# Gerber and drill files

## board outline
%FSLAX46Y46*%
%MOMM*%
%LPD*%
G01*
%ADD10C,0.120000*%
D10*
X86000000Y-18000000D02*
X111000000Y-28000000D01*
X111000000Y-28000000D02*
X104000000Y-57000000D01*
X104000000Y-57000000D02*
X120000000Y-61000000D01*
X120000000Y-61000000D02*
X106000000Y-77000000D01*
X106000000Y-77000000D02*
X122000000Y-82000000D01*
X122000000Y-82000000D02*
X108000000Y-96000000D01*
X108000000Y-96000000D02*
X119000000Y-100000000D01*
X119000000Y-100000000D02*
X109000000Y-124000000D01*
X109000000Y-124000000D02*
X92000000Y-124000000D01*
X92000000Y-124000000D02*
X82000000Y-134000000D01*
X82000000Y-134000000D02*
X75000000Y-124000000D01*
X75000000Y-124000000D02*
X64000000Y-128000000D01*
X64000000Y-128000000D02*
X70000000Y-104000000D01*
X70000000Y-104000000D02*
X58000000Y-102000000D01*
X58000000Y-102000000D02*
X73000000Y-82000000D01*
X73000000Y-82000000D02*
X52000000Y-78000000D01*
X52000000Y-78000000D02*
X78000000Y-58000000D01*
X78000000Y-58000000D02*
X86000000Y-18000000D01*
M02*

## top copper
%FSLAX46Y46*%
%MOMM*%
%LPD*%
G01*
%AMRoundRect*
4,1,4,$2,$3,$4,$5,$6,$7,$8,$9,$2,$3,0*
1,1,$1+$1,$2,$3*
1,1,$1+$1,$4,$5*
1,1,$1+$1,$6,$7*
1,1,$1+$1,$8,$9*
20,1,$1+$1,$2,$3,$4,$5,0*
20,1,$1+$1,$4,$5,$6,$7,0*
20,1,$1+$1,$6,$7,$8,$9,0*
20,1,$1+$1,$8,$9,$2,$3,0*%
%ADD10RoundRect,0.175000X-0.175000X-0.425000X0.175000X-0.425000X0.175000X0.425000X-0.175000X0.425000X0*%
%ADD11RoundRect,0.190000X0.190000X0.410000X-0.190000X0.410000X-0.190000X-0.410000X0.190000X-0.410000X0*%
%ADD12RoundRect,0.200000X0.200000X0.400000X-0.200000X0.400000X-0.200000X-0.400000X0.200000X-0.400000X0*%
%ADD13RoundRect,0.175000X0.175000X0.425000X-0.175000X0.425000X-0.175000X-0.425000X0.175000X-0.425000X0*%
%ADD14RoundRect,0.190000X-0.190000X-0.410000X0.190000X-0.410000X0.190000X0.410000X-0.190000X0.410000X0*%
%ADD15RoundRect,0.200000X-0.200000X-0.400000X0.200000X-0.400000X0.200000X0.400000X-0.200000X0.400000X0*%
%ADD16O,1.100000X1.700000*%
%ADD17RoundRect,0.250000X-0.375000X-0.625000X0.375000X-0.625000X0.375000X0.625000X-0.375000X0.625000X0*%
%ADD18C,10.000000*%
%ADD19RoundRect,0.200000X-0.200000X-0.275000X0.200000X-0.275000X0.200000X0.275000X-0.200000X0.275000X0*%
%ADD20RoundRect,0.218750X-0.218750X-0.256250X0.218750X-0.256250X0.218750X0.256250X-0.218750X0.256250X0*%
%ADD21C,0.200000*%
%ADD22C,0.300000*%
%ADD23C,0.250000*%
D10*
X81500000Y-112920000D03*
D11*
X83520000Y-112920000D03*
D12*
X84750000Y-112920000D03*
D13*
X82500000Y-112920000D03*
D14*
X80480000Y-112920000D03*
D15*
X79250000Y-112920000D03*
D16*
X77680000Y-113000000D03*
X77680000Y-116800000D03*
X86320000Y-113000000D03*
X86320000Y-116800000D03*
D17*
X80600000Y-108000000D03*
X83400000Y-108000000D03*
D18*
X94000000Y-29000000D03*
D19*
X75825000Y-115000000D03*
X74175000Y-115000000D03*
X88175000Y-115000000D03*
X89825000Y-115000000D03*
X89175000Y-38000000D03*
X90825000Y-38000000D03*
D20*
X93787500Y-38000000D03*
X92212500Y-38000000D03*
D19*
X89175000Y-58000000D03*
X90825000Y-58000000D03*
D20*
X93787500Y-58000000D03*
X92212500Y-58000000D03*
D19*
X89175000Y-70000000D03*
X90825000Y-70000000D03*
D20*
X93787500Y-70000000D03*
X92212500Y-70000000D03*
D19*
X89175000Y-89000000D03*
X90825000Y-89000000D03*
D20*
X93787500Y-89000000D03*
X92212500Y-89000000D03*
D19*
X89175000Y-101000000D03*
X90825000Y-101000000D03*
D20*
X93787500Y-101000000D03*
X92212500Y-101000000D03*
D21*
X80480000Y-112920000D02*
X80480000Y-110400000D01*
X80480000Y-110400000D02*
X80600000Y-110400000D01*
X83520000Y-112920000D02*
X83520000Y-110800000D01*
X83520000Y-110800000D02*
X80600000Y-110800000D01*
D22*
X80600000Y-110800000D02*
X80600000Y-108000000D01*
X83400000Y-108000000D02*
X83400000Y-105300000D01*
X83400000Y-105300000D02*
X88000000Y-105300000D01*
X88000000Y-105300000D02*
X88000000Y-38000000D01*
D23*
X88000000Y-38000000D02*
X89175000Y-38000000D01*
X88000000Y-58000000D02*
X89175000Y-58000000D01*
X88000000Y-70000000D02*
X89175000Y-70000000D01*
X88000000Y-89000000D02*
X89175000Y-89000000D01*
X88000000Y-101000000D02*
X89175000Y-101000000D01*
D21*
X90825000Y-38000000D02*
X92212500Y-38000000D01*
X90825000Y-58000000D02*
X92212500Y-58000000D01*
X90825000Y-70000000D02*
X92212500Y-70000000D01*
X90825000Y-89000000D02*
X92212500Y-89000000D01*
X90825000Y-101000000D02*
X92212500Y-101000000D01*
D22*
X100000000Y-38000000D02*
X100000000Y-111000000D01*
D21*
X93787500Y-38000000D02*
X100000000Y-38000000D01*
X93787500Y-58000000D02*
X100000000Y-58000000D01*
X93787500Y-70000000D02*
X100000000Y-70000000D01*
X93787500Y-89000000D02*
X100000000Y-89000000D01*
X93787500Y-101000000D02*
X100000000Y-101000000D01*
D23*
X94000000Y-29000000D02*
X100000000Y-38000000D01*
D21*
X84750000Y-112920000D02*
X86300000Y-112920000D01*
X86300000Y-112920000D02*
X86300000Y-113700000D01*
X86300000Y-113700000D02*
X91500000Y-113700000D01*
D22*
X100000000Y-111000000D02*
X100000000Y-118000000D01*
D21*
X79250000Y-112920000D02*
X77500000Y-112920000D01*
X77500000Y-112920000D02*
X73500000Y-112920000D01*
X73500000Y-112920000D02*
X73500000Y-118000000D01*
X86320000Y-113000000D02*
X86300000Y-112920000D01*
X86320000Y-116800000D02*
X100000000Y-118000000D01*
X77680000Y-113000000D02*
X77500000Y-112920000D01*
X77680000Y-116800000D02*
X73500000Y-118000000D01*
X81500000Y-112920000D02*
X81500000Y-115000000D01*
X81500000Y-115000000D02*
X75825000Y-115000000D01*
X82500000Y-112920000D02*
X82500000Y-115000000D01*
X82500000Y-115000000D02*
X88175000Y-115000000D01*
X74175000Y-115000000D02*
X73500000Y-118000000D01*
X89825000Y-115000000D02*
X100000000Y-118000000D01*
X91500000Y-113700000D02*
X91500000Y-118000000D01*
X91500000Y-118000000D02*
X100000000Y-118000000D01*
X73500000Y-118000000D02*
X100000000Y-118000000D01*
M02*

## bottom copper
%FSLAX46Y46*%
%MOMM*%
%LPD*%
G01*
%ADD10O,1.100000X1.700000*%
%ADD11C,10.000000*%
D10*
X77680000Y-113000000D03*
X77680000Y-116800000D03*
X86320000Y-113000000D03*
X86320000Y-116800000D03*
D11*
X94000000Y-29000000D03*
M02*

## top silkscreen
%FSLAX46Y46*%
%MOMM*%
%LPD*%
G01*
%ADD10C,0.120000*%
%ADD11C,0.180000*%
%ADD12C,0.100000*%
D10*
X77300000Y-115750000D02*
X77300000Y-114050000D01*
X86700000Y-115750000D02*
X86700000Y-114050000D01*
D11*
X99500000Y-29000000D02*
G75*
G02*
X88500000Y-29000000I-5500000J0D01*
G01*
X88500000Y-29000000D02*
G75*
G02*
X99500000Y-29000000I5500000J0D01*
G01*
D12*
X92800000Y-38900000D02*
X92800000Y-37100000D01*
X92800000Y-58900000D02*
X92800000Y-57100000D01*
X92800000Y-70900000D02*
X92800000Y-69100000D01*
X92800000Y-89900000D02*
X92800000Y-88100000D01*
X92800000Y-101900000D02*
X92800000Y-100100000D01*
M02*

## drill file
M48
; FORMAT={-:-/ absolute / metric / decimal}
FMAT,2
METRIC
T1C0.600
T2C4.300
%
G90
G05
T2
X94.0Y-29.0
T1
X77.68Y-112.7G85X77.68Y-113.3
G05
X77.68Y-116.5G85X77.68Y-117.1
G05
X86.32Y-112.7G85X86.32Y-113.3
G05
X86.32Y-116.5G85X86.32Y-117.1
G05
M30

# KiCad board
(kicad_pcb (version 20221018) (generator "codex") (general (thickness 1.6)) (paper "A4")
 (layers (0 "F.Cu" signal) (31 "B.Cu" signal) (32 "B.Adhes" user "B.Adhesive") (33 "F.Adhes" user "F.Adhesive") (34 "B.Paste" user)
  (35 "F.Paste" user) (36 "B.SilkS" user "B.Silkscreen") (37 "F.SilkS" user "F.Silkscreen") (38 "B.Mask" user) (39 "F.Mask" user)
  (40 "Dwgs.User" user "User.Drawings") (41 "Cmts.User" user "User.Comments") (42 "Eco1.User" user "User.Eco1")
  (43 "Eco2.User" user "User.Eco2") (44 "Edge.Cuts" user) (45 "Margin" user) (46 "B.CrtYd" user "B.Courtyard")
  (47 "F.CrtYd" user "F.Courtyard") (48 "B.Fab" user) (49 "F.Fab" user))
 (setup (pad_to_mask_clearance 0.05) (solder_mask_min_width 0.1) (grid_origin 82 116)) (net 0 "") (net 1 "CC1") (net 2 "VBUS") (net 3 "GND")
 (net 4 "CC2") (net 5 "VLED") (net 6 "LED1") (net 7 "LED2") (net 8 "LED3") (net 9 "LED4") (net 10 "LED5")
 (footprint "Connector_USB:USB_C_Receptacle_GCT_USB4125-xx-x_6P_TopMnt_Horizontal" (layer "F.Cu") (at 82 116)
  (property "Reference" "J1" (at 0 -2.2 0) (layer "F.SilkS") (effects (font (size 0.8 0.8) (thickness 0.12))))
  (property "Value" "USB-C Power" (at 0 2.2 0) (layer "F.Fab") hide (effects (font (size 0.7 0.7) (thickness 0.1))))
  (fp_line (start -4.7 -0.25) (end -4.7 -1.95) (stroke (width 0.12) (type solid)) (layer "F.SilkS"))
  (fp_line (start 4.7 -0.25) (end 4.7 -1.95) (stroke (width 0.12) (type solid)) (layer "F.SilkS"))
  (pad "A5" smd roundrect (at -0.5 -3.08) (size 0.7 1.2) (layers "F.Cu" "F.Paste" "F.Mask") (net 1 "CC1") (roundrect_rratio 0.25))
  (pad "A9" smd roundrect (at 1.52 -3.08 180) (size 0.76 1.2) (layers "F.Cu" "F.Paste" "F.Mask") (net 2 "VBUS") (roundrect_rratio 0.25))
  (pad "A12" smd roundrect (at 2.75 -3.08 180) (size 0.8 1.2) (layers "F.Cu" "F.Paste" "F.Mask") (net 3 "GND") (roundrect_rratio 0.25))
  (pad "B5" smd roundrect (at 0.5 -3.08 180) (size 0.7 1.2) (layers "F.Cu" "F.Paste" "F.Mask") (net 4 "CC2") (roundrect_rratio 0.25))
  (pad "B9" smd roundrect (at -1.52 -3.08) (size 0.76 1.2) (layers "F.Cu" "F.Paste" "F.Mask") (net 2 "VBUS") (roundrect_rratio 0.25))
  (pad "B12" smd roundrect (at -2.75 -3.08) (size 0.8 1.2) (layers "F.Cu" "F.Paste" "F.Mask") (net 3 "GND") (roundrect_rratio 0.25))
  (pad "SH" thru_hole oval (at -4.32 -3) (size 1.1 1.7) (drill oval 0.6 1.2) (layers "*.Cu" "*.Mask") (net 3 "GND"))
  (pad "SH" thru_hole oval (at -4.32 0.8) (size 1.1 1.7) (drill oval 0.6 1.2) (layers "*.Cu" "*.Mask") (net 3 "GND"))
  (pad "SH" thru_hole oval (at 4.32 -3) (size 1.1 1.7) (drill oval 0.6 1.2) (layers "*.Cu" "*.Mask") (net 3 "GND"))
  (pad "SH" thru_hole oval (at 4.32 0.8) (size 1.1 1.7) (drill oval 0.6 1.2) (layers "*.Cu" "*.Mask") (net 3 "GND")))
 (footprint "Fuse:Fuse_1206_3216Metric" (layer "F.Cu") (at 82 108)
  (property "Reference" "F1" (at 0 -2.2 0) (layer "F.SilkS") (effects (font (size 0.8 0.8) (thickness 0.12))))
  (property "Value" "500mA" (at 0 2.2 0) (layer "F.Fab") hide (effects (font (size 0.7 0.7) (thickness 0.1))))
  (pad "1" smd roundrect (at -1.4 0) (size 1.25 1.75) (layers "F.Cu" "F.Paste" "F.Mask") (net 2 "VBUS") (roundrect_rratio 0.2))
  (pad "2" smd roundrect (at 1.4 0) (size 1.25 1.75) (layers "F.Cu" "F.Paste" "F.Mask") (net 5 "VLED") (roundrect_rratio 0.2)))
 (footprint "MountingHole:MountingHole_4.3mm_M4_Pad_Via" (layer "F.Cu") (at 94 29)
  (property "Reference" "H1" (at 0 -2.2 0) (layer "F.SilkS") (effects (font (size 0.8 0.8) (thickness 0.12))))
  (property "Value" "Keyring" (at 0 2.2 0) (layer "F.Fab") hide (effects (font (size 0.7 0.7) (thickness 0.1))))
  (fp_circle (center 0 0) (end 5.5 0) (stroke (width 0.18) (type solid)) (fill none) (layer "F.SilkS"))
  (pad "1" thru_hole circle (at 0 0) (size 10 10) (drill 4.3) (layers "*.Cu" "*.Mask") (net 3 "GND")))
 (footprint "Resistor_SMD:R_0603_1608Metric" (layer "F.Cu") (at 75 115 180)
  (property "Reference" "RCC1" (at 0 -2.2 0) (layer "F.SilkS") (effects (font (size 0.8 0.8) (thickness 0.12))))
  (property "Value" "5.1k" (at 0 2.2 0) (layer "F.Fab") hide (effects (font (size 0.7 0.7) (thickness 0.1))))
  (pad "1" smd roundrect (at -0.825 0) (size 0.8 0.95) (layers "F.Cu" "F.Paste" "F.Mask") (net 1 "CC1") (roundrect_rratio 0.25))
  (pad "2" smd roundrect (at 0.825 0) (size 0.8 0.95) (layers "F.Cu" "F.Paste" "F.Mask") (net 3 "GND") (roundrect_rratio 0.25)))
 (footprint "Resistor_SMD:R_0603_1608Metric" (layer "F.Cu") (at 89 115 0)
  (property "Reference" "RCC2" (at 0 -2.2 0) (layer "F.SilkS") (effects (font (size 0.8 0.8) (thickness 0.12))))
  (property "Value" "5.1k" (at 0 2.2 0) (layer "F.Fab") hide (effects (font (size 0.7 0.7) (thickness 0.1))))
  (pad "1" smd roundrect (at -0.825 0) (size 0.8 0.95) (layers "F.Cu" "F.Paste" "F.Mask") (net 4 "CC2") (roundrect_rratio 0.25))
  (pad "2" smd roundrect (at 0.825 0) (size 0.8 0.95) (layers "F.Cu" "F.Paste" "F.Mask") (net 3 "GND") (roundrect_rratio 0.25)))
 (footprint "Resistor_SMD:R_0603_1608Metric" (layer "F.Cu") (at 90 38 0)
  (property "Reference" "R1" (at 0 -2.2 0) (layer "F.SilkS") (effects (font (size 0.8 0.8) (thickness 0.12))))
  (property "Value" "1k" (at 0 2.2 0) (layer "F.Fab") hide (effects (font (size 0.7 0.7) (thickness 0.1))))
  (pad "1" smd roundrect (at -0.825 0) (size 0.8 0.95) (layers "F.Cu" "F.Paste" "F.Mask") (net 5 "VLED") (roundrect_rratio 0.25))
  (pad "2" smd roundrect (at 0.825 0) (size 0.8 0.95) (layers "F.Cu" "F.Paste" "F.Mask") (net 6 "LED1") (roundrect_rratio 0.25)))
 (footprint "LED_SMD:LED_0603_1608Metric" (layer "F.Cu") (at 93 38 180)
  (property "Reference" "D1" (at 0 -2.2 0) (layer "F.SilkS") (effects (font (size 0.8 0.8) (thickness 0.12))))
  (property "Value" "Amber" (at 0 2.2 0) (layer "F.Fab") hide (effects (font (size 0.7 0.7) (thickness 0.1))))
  (fp_line (start 0.2 -0.9) (end 0.2 0.9) (stroke (width 0.1) (type solid)) (layer "F.SilkS"))
  (pad "1" smd roundrect (at -0.7875 0) (size 0.875 0.95) (layers "F.Cu" "F.Paste" "F.Mask") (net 3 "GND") (roundrect_rratio 0.25))
  (pad "2" smd roundrect (at 0.7875 0) (size 0.875 0.95) (layers "F.Cu" "F.Paste" "F.Mask") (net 6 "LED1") (roundrect_rratio 0.25)))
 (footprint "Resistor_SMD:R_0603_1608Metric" (layer "F.Cu") (at 90 58 0)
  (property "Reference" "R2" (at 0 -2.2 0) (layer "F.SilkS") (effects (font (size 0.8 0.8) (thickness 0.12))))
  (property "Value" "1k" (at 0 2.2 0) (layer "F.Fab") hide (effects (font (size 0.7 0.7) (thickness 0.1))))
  (pad "1" smd roundrect (at -0.825 0) (size 0.8 0.95) (layers "F.Cu" "F.Paste" "F.Mask") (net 5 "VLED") (roundrect_rratio 0.25))
  (pad "2" smd roundrect (at 0.825 0) (size 0.8 0.95) (layers "F.Cu" "F.Paste" "F.Mask") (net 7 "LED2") (roundrect_rratio 0.25)))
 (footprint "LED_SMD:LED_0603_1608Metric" (layer "F.Cu") (at 93 58 180)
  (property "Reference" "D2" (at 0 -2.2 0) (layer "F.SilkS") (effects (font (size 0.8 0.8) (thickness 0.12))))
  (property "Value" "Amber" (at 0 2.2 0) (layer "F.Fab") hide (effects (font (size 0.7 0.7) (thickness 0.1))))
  (fp_line (start 0.2 -0.9) (end 0.2 0.9) (stroke (width 0.1) (type solid)) (layer "F.SilkS"))
  (pad "1" smd roundrect (at -0.7875 0) (size 0.875 0.95) (layers "F.Cu" "F.Paste" "F.Mask") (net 3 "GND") (roundrect_rratio 0.25))
  (pad "2" smd roundrect (at 0.7875 0) (size 0.875 0.95) (layers "F.Cu" "F.Paste" "F.Mask") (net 7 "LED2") (roundrect_rratio 0.25)))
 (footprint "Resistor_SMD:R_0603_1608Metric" (layer "F.Cu") (at 90 70 0)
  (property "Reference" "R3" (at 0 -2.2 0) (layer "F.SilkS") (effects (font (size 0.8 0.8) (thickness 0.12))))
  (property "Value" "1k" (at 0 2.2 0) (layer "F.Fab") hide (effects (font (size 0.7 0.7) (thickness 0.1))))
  (pad "1" smd roundrect (at -0.825 0) (size 0.8 0.95) (layers "F.Cu" "F.Paste" "F.Mask") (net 5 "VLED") (roundrect_rratio 0.25))
  (pad "2" smd roundrect (at 0.825 0) (size 0.8 0.95) (layers "F.Cu" "F.Paste" "F.Mask") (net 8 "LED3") (roundrect_rratio 0.25)))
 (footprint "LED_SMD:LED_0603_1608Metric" (layer "F.Cu") (at 93 70 180)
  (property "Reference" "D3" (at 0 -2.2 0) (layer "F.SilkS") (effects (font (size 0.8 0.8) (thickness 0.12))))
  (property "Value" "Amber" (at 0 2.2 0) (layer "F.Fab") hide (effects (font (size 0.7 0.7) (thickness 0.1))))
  (fp_line (start 0.2 -0.9) (end 0.2 0.9) (stroke (width 0.1) (type solid)) (layer "F.SilkS"))
  (pad "1" smd roundrect (at -0.7875 0) (size 0.875 0.95) (layers "F.Cu" "F.Paste" "F.Mask") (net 3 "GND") (roundrect_rratio 0.25))
  (pad "2" smd roundrect (at 0.7875 0) (size 0.875 0.95) (layers "F.Cu" "F.Paste" "F.Mask") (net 8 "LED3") (roundrect_rratio 0.25)))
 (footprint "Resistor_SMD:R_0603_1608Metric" (layer "F.Cu") (at 90 89 0)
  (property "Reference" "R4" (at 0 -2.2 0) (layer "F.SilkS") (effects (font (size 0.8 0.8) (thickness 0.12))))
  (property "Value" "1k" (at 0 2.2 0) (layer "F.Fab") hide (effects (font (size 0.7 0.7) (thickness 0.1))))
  (pad "1" smd roundrect (at -0.825 0) (size 0.8 0.95) (layers "F.Cu" "F.Paste" "F.Mask") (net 5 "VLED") (roundrect_rratio 0.25))
  (pad "2" smd roundrect (at 0.825 0) (size 0.8 0.95) (layers "F.Cu" "F.Paste" "F.Mask") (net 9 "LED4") (roundrect_rratio 0.25)))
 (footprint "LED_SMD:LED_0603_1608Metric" (layer "F.Cu") (at 93 89 180)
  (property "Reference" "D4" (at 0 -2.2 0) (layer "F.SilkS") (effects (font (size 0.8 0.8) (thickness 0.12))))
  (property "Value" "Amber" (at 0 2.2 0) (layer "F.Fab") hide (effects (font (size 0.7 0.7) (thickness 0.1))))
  (fp_line (start 0.2 -0.9) (end 0.2 0.9) (stroke (width 0.1) (type solid)) (layer "F.SilkS"))
  (pad "1" smd roundrect (at -0.7875 0) (size 0.875 0.95) (layers "F.Cu" "F.Paste" "F.Mask") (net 3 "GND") (roundrect_rratio 0.25))
  (pad "2" smd roundrect (at 0.7875 0) (size 0.875 0.95) (layers "F.Cu" "F.Paste" "F.Mask") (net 9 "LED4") (roundrect_rratio 0.25)))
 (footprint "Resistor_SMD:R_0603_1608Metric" (layer "F.Cu") (at 90 101 0)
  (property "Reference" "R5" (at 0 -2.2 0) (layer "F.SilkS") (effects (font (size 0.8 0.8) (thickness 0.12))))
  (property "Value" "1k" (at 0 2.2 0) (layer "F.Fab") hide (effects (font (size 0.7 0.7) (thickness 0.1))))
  (pad "1" smd roundrect (at -0.825 0) (size 0.8 0.95) (layers "F.Cu" "F.Paste" "F.Mask") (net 5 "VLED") (roundrect_rratio 0.25))
  (pad "2" smd roundrect (at 0.825 0) (size 0.8 0.95) (layers "F.Cu" "F.Paste" "F.Mask") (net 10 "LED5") (roundrect_rratio 0.25)))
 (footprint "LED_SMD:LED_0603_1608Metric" (layer "F.Cu") (at 93 101 180)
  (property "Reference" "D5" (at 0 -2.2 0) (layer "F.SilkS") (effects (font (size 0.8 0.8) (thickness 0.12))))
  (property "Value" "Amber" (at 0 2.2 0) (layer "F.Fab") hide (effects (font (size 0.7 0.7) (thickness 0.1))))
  (fp_line (start 0.2 -0.9) (end 0.2 0.9) (stroke (width 0.1) (type solid)) (layer "F.SilkS"))
  (pad "1" smd roundrect (at -0.7875 0) (size 0.875 0.95) (layers "F.Cu" "F.Paste" "F.Mask") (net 3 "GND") (roundrect_rratio 0.25))
  (pad "2" smd roundrect (at 0.7875 0) (size 0.875 0.95) (layers "F.Cu" "F.Paste" "F.Mask") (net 10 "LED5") (roundrect_rratio 0.25)))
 (gr_line (start 86 18) (end 111 28) (stroke (width 0.12) (type solid)) (layer "Edge.Cuts"))
 (gr_line (start 111 28) (end 104 57) (stroke (width 0.12) (type solid)) (layer "Edge.Cuts"))
 (gr_line (start 104 57) (end 120 61) (stroke (width 0.12) (type solid)) (layer "Edge.Cuts"))
 (gr_line (start 120 61) (end 106 77) (stroke (width 0.12) (type solid)) (layer "Edge.Cuts"))
 (gr_line (start 106 77) (end 122 82) (stroke (width 0.12) (type solid)) (layer "Edge.Cuts"))
 (gr_line (start 122 82) (end 108 96) (stroke (width 0.12) (type solid)) (layer "Edge.Cuts"))
 (gr_line (start 108 96) (end 119 100) (stroke (width 0.12) (type solid)) (layer "Edge.Cuts"))
 (gr_line (start 119 100) (end 109 124) (stroke (width 0.12) (type solid)) (layer "Edge.Cuts"))
 (gr_line (start 109 124) (end 92 124) (stroke (width 0.12) (type solid)) (layer "Edge.Cuts"))
 (gr_line (start 92 124) (end 82 134) (stroke (width 0.12) (type solid)) (layer "Edge.Cuts"))
 (gr_line (start 82 134) (end 75 124) (stroke (width 0.12) (type solid)) (layer "Edge.Cuts"))
 (gr_line (start 75 124) (end 64 128) (stroke (width 0.12) (type solid)) (layer "Edge.Cuts"))
 (gr_line (start 64 128) (end 70 104) (stroke (width 0.12) (type solid)) (layer "Edge.Cuts"))
 (gr_line (start 70 104) (end 58 102) (stroke (width 0.12) (type solid)) (layer "Edge.Cuts"))
 (gr_line (start 58 102) (end 73 82) (stroke (width 0.12) (type solid)) (layer "Edge.Cuts"))
 (gr_line (start 73 82) (end 52 78) (stroke (width 0.12) (type solid)) (layer "Edge.Cuts"))
 (gr_line (start 52 78) (end 78 58) (stroke (width 0.12) (type solid)) (layer "Edge.Cuts"))
 (gr_line (start 78 58) (end 86 18) (stroke (width 0.12) (type solid)) (layer "Edge.Cuts"))
 (segment (start 80.48 112.92) (end 80.48 110.4) (width 0.20) (layer "F.Cu") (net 2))
 (segment (start 80.48 110.4) (end 80.6 110.4) (width 0.20) (layer "F.Cu") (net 2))
 (segment (start 83.52 112.92) (end 83.52 110.8) (width 0.20) (layer "F.Cu") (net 2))
 (segment (start 83.52 110.8) (end 80.6 110.8) (width 0.20) (layer "F.Cu") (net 2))
 (segment (start 80.6 110.8) (end 80.6 108) (width 0.30) (layer "F.Cu") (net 2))
 (segment (start 83.4 108) (end 83.4 105.3) (width 0.30) (layer "F.Cu") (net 5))
 (segment (start 83.4 105.3) (end 88 105.3) (width 0.30) (layer "F.Cu") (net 5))
 (segment (start 88 105.3) (end 88 38) (width 0.30) (layer "F.Cu") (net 5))
 (segment (start 88 38) (end 89.175 38) (width 0.25) (layer "F.Cu") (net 5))
 (segment (start 88 58) (end 89.175 58) (width 0.25) (layer "F.Cu") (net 5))
 (segment (start 88 70) (end 89.175 70) (width 0.25) (layer "F.Cu") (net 5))
 (segment (start 88 89) (end 89.175 89) (width 0.25) (layer "F.Cu") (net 5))
 (segment (start 88 101) (end 89.175 101) (width 0.25) (layer "F.Cu") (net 5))
 (segment (start 90.825 38) (end 92.2125 38) (width 0.20) (layer "F.Cu") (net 6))
 (segment (start 90.825 58) (end 92.2125 58) (width 0.20) (layer "F.Cu") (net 7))
 (segment (start 90.825 70) (end 92.2125 70) (width 0.20) (layer "F.Cu") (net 8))
 (segment (start 90.825 89) (end 92.2125 89) (width 0.20) (layer "F.Cu") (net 9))
 (segment (start 90.825 101) (end 92.2125 101) (width 0.20) (layer "F.Cu") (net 10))
 (segment (start 100 38) (end 100 111) (width 0.30) (layer "F.Cu") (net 3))
 (segment (start 93.7875 38) (end 100 38) (width 0.20) (layer "F.Cu") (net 3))
 (segment (start 93.7875 58) (end 100 58) (width 0.20) (layer "F.Cu") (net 3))
 (segment (start 93.7875 70) (end 100 70) (width 0.20) (layer "F.Cu") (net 3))
 (segment (start 93.7875 89) (end 100 89) (width 0.20) (layer "F.Cu") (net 3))
 (segment (start 93.7875 101) (end 100 101) (width 0.20) (layer "F.Cu") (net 3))
 (segment (start 94 29) (end 100 38) (width 0.25) (layer "F.Cu") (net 3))
 (segment (start 84.75 112.92) (end 86.3 112.92) (width 0.20) (layer "F.Cu") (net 3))
 (segment (start 86.3 112.92) (end 86.3 113.7) (width 0.20) (layer "F.Cu") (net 3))
 (segment (start 86.3 113.7) (end 91.5 113.7) (width 0.20) (layer "F.Cu") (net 3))
 (segment (start 100 111) (end 100 118) (width 0.30) (layer "F.Cu") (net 3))
 (segment (start 79.25 112.92) (end 77.5 112.92) (width 0.20) (layer "F.Cu") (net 3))
 (segment (start 77.5 112.92) (end 73.5 112.92) (width 0.20) (layer "F.Cu") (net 3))
 (segment (start 73.5 112.92) (end 73.5 118) (width 0.20) (layer "F.Cu") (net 3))
 (segment (start 86.32 113) (end 86.3 112.92) (width 0.20) (layer "F.Cu") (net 3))
 (segment (start 86.32 116.8) (end 100 118) (width 0.20) (layer "F.Cu") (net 3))
 (segment (start 77.68 113) (end 77.5 112.92) (width 0.20) (layer "F.Cu") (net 3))
 (segment (start 77.68 116.8) (end 73.5 118) (width 0.20) (layer "F.Cu") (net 3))
 (segment (start 81.5 112.92) (end 81.5 115) (width 0.20) (layer "F.Cu") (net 1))
 (segment (start 81.5 115) (end 75.825 115) (width 0.20) (layer "F.Cu") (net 1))
 (segment (start 82.5 112.92) (end 82.5 115) (width 0.20) (layer "F.Cu") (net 4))
 (segment (start 82.5 115) (end 88.175 115) (width 0.20) (layer "F.Cu") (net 4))
 (segment (start 74.175 115) (end 73.5 118) (width 0.20) (layer "F.Cu") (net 3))
 (segment (start 89.825 115) (end 100 118) (width 0.20) (layer "F.Cu") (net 3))
 (segment (start 91.5 113.7) (end 91.5 118) (width 0.20) (layer "F.Cu") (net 3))
 (segment (start 91.5 118) (end 100 118) (width 0.20) (layer "F.Cu") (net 3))
 (segment (start 73.5 118) (end 100 118) (width 0.20) (layer "F.Cu") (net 3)))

